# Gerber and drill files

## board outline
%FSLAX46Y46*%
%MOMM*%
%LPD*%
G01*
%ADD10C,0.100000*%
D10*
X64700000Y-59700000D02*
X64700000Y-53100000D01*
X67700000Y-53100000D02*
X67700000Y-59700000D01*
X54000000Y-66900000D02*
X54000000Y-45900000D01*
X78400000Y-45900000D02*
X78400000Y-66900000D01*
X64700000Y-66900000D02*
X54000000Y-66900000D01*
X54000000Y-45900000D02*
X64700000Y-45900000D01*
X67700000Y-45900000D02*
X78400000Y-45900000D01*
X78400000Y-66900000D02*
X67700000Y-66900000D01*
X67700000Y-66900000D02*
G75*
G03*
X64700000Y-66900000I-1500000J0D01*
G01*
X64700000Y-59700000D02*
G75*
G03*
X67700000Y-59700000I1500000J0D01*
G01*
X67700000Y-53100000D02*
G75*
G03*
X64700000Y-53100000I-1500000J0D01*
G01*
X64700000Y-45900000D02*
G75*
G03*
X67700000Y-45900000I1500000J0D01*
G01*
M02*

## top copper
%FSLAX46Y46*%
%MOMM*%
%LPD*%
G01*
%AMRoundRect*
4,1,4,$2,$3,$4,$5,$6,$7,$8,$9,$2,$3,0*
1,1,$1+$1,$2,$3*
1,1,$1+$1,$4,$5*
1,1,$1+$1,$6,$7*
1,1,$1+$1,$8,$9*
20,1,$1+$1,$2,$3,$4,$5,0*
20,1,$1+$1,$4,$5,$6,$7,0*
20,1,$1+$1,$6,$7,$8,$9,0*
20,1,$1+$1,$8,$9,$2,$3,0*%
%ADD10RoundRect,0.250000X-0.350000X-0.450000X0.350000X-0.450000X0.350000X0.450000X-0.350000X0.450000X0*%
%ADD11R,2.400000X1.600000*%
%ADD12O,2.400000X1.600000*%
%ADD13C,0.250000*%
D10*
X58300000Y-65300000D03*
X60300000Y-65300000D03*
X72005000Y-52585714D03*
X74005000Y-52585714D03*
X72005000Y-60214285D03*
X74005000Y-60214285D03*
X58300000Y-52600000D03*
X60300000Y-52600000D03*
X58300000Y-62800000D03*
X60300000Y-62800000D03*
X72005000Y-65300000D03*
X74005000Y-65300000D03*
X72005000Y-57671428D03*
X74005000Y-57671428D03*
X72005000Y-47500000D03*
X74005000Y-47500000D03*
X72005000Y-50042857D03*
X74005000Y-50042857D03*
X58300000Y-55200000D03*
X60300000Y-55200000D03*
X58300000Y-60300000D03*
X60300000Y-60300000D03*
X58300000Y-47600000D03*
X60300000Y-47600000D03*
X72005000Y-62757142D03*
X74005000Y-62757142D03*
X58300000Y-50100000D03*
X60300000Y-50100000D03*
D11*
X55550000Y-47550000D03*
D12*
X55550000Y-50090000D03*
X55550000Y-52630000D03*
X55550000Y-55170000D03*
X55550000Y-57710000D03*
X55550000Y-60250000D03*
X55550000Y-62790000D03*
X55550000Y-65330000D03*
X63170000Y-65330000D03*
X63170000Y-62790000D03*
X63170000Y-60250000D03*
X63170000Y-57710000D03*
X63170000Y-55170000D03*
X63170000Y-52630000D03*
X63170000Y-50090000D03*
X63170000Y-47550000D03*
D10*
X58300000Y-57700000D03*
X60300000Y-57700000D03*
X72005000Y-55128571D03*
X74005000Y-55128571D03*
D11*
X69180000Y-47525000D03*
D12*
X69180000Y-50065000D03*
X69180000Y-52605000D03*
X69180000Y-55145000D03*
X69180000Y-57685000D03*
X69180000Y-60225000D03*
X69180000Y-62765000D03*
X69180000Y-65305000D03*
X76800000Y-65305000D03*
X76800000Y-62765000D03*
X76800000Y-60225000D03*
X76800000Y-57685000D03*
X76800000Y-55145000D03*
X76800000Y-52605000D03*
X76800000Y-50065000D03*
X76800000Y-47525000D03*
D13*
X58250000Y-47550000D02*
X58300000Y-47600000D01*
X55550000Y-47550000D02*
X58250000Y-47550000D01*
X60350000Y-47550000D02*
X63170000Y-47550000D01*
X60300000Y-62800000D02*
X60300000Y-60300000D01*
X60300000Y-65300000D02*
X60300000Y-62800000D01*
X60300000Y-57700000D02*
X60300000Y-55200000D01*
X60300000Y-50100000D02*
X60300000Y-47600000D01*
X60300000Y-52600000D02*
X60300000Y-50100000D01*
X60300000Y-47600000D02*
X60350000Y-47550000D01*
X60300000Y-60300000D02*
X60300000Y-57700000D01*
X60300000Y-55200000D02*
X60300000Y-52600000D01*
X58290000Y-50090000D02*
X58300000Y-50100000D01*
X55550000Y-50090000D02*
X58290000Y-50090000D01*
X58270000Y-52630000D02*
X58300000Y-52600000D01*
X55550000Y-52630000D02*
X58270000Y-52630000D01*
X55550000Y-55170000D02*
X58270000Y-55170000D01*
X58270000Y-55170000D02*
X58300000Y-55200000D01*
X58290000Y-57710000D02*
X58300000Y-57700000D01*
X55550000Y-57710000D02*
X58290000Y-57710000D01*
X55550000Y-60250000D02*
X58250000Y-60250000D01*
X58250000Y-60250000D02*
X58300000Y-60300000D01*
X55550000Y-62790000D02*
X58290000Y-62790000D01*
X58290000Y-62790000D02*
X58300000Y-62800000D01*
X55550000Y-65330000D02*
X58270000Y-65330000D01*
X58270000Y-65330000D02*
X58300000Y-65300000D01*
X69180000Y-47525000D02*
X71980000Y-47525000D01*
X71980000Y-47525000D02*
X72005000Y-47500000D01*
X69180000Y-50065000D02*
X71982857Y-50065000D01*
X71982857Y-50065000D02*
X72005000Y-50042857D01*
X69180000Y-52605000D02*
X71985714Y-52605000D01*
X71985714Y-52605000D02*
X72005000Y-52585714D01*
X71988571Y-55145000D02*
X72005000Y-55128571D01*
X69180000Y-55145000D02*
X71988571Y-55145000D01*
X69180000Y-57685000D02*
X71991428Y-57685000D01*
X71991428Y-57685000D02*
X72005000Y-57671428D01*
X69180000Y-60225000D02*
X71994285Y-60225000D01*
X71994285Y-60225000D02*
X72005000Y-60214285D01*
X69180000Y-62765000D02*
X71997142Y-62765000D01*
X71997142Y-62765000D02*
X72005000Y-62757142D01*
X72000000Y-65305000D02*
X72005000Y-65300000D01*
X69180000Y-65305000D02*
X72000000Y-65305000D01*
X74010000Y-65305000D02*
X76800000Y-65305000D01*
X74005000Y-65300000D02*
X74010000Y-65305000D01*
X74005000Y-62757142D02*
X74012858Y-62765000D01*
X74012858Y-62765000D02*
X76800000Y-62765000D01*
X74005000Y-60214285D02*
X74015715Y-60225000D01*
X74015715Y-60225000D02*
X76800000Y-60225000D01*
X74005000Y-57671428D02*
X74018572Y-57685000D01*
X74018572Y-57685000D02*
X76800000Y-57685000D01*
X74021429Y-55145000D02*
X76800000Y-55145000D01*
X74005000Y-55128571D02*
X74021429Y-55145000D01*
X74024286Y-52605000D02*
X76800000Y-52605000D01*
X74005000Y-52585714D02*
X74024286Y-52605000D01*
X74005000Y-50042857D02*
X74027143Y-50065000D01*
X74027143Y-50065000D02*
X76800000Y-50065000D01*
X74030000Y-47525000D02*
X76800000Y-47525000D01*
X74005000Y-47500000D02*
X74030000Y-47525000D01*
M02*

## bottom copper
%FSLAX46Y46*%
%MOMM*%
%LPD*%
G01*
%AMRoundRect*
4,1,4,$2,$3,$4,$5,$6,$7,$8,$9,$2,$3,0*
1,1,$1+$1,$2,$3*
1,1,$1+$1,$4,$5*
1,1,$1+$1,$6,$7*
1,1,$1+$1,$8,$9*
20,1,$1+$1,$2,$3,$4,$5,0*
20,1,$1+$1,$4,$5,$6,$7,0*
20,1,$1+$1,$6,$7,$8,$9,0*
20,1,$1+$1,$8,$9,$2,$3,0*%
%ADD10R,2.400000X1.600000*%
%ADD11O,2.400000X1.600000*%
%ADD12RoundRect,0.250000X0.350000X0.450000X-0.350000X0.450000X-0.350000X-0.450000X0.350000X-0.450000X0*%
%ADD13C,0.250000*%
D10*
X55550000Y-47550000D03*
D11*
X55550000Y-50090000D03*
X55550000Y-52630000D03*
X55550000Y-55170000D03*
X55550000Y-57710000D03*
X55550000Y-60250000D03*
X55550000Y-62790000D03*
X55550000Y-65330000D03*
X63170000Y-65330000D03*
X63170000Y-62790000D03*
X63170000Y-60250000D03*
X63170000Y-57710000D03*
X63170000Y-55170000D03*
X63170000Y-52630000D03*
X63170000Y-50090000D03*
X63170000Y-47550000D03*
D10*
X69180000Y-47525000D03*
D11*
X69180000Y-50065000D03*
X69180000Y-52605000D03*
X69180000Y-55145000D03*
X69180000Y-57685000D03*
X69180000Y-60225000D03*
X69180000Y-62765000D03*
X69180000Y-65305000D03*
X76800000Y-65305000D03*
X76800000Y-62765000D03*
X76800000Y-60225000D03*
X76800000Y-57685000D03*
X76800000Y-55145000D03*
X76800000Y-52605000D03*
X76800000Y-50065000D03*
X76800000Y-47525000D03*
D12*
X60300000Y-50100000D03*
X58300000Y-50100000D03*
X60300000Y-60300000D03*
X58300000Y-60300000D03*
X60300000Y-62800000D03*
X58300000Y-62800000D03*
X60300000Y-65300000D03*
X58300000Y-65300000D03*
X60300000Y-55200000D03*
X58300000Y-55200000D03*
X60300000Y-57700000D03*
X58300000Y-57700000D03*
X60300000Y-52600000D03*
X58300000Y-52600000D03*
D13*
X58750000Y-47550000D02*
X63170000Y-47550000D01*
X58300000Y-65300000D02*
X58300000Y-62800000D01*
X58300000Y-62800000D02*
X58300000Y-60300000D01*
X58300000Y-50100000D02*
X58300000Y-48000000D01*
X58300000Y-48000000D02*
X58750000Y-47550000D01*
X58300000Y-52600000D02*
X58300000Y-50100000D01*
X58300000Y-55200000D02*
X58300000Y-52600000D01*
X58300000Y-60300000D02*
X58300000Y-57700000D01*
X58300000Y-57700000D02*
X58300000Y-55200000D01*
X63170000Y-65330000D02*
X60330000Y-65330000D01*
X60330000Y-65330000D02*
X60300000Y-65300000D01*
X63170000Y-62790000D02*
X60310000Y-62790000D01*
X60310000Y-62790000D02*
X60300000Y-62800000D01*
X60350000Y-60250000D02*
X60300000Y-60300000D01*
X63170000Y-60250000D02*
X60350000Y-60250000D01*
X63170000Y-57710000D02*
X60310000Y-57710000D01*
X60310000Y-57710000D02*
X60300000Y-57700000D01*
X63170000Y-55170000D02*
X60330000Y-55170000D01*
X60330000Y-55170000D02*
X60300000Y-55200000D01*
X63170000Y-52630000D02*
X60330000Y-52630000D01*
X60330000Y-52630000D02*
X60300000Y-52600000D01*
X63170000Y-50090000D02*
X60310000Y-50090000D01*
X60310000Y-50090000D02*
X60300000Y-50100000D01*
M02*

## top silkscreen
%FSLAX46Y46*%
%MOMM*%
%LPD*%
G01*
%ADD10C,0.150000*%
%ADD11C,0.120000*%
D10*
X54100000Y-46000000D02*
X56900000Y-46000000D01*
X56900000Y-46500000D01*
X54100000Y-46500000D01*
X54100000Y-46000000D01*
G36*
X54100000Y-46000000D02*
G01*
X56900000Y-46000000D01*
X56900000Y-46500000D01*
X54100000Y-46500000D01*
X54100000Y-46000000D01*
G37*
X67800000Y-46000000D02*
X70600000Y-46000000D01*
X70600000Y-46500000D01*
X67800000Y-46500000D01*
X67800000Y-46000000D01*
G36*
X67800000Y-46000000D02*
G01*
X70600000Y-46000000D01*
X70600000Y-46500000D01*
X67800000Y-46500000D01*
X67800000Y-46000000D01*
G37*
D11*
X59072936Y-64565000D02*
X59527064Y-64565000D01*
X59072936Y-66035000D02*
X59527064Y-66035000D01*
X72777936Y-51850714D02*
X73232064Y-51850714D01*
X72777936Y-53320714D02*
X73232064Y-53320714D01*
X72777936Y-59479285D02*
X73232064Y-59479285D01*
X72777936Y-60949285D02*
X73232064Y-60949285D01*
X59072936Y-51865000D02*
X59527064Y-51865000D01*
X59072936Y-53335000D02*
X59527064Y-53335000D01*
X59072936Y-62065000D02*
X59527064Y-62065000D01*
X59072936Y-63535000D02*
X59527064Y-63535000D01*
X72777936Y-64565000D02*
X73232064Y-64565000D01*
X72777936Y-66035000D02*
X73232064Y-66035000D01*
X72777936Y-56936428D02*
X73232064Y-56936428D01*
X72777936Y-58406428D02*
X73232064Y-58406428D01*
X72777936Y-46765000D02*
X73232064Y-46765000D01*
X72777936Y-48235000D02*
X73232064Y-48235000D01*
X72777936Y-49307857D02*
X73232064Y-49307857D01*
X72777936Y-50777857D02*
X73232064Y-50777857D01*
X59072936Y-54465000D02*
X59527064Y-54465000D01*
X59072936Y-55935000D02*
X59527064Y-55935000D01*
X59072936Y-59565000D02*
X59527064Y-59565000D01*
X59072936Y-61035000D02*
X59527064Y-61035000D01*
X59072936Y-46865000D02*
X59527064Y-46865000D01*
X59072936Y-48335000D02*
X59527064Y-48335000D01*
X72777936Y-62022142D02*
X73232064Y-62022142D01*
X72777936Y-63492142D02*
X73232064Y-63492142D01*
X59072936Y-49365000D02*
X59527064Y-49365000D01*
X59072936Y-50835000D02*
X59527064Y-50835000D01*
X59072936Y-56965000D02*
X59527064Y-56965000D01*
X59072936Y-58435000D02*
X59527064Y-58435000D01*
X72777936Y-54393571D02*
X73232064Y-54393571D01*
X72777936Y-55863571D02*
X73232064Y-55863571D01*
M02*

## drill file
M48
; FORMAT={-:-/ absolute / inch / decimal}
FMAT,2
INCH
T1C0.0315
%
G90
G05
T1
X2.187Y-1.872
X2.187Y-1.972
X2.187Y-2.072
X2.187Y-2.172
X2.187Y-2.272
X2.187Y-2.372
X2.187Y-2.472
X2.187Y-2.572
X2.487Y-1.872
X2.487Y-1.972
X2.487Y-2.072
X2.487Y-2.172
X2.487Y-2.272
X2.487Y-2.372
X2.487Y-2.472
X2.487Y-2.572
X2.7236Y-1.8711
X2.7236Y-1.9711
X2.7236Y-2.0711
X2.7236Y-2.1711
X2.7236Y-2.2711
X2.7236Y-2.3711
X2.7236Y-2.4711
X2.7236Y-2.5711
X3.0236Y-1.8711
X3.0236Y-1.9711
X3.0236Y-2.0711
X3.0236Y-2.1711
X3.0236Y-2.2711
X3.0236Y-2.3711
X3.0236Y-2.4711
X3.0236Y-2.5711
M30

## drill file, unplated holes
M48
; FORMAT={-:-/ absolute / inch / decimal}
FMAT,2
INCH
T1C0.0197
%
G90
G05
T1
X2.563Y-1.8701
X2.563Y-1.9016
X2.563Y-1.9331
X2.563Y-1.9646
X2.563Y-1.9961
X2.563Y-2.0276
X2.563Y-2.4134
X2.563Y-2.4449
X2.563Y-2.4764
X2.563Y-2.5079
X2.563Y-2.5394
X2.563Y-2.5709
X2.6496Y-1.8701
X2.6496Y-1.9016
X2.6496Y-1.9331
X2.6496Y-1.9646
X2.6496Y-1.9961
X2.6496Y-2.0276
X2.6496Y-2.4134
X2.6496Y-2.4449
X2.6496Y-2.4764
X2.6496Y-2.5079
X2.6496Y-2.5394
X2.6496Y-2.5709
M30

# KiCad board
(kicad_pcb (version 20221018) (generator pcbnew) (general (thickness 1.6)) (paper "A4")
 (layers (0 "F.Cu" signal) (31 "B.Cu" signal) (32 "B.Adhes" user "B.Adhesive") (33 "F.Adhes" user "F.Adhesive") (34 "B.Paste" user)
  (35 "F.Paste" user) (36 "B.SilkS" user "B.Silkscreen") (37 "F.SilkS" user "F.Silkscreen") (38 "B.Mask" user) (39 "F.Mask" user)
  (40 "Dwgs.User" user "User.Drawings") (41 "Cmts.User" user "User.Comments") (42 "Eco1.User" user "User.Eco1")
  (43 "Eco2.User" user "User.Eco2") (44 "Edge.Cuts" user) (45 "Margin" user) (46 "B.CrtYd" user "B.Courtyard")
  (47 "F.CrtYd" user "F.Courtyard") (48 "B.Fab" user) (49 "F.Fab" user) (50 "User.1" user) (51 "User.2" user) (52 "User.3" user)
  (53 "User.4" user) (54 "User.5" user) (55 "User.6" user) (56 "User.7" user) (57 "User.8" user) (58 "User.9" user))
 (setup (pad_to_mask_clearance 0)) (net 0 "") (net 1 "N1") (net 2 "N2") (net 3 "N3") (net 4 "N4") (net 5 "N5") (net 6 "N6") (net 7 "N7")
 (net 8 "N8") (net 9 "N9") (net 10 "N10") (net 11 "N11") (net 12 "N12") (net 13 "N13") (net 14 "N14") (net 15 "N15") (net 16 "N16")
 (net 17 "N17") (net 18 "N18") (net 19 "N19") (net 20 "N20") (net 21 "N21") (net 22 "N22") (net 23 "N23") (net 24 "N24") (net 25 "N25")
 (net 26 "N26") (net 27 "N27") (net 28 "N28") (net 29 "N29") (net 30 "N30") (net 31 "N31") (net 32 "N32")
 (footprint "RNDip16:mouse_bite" (layer "F.Cu") (at 66.2 63.3 90)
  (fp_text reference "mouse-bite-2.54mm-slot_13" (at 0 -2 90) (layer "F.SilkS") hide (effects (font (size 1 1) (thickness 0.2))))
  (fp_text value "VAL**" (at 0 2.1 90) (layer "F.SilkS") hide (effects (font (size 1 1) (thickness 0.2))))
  (fp_arc (start -3.6 -1.5) (mid -2.1 0) (end -3.6 1.5) (stroke (width 0.1) (type solid)) (layer "Edge.Cuts"))
  (fp_arc (start 3.6 1.5) (mid 2.1 0) (end 3.6 -1.5) (stroke (width 0.1) (type solid)) (layer "Edge.Cuts"))
  (pad "" np_thru_hole circle (at -2 -1.1 90) (size 0.5 0.5) (drill 0.5) (layers "F&B.Cu" "*.Mask"))
  (pad "" np_thru_hole circle (at -2 1.1 90) (size 0.5 0.5) (drill 0.5) (layers "F&B.Cu" "*.Mask"))
  (pad "" np_thru_hole circle (at -1.2 -1.1 90) (size 0.5 0.5) (drill 0.5) (layers "F&B.Cu" "*.Mask"))
  (pad "" np_thru_hole circle (at -1.2 1.1 90) (size 0.5 0.5) (drill 0.5) (layers "F&B.Cu" "*.Mask"))
  (pad "" np_thru_hole circle (at -0.4 -1.1 90) (size 0.5 0.5) (drill 0.5) (layers "F&B.Cu" "*.Mask"))
  (pad "" np_thru_hole circle (at -0.4 1.1 90) (size 0.5 0.5) (drill 0.5) (layers "F&B.Cu" "*.Mask"))
  (pad "" np_thru_hole circle (at 0.4 -1.1 90) (size 0.5 0.5) (drill 0.5) (layers "F&B.Cu" "*.Mask"))
  (pad "" np_thru_hole circle (at 0.4 1.1 90) (size 0.5 0.5) (drill 0.5) (layers "F&B.Cu" "*.Mask"))
  (pad "" np_thru_hole circle (at 1.2 -1.1 90) (size 0.5 0.5) (drill 0.5) (layers "F&B.Cu" "*.Mask"))
  (pad "" np_thru_hole circle (at 1.2 1.1 90) (size 0.5 0.5) (drill 0.5) (layers "F&B.Cu" "*.Mask"))
  (pad "" np_thru_hole circle (at 2 -1.1 90) (size 0.5 0.5) (drill 0.5) (layers "F&B.Cu" "*.Mask"))
  (pad "" np_thru_hole circle (at 2 1.1 90) (size 0.5 0.5) (drill 0.5) (layers "F&B.Cu" "*.Mask")))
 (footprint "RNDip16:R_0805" (layer "F.Cu") (at 59.3 65.3)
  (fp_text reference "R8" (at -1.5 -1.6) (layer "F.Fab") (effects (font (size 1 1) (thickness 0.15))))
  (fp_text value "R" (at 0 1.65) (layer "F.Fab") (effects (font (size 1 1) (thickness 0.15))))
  (fp_line (start -0.227064 -0.735) (end 0.227064 -0.735) (stroke (width 0.12) (type solid)) (layer "F.SilkS"))
  (fp_line (start -0.227064 0.735) (end 0.227064 0.735) (stroke (width 0.12) (type solid)) (layer "F.SilkS"))
  (pad "1" smd roundrect (at -1 0) (size 1.2 1.4) (layers "F.Cu" "F.Paste" "F.Mask") (roundrect_rratio 0.2083333333) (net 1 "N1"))
  (pad "2" smd roundrect (at 1 0) (size 1.2 1.4) (layers "F.Cu" "F.Paste" "F.Mask") (roundrect_rratio 0.2083333333) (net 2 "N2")))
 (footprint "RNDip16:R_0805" (layer "F.Cu") (at 73.005 52.585714)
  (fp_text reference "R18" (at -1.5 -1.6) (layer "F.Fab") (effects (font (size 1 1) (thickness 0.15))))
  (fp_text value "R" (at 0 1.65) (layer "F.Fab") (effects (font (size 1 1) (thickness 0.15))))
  (fp_line (start -0.227064 -0.735) (end 0.227064 -0.735) (stroke (width 0.12) (type solid)) (layer "F.SilkS"))
  (fp_line (start -0.227064 0.735) (end 0.227064 0.735) (stroke (width 0.12) (type solid)) (layer "F.SilkS"))
  (pad "1" smd roundrect (at -1 0) (size 1.2 1.4) (layers "F.Cu" "F.Paste" "F.Mask") (roundrect_rratio 0.2083333333) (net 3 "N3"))
  (pad "2" smd roundrect (at 1 0) (size 1.2 1.4) (layers "F.Cu" "F.Paste" "F.Mask") (roundrect_rratio 0.2083333333) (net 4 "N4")))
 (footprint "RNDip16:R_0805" (layer "F.Cu") (at 73.005 60.214285)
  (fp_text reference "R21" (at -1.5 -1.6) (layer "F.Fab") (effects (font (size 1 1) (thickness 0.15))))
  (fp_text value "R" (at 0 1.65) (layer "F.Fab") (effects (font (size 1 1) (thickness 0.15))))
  (fp_line (start -0.227064 -0.735) (end 0.227064 -0.735) (stroke (width 0.12) (type solid)) (layer "F.SilkS"))
  (fp_line (start -0.227064 0.735) (end 0.227064 0.735) (stroke (width 0.12) (type solid)) (layer "F.SilkS"))
  (pad "1" smd roundrect (at -1 0) (size 1.2 1.4) (layers "F.Cu" "F.Paste" "F.Mask") (roundrect_rratio 0.2083333333) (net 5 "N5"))
  (pad "2" smd roundrect (at 1 0) (size 1.2 1.4) (layers "F.Cu" "F.Paste" "F.Mask") (roundrect_rratio 0.2083333333) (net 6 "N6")))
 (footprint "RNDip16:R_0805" (layer "F.Cu") (at 59.3 52.6)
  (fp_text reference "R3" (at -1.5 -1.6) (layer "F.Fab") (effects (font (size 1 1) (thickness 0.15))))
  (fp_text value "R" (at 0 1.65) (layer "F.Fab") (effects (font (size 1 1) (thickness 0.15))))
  (fp_line (start -0.227064 -0.735) (end 0.227064 -0.735) (stroke (width 0.12) (type solid)) (layer "F.SilkS"))
  (fp_line (start -0.227064 0.735) (end 0.227064 0.735) (stroke (width 0.12) (type solid)) (layer "F.SilkS"))
  (pad "1" smd roundrect (at -1 0) (size 1.2 1.4) (layers "F.Cu" "F.Paste" "F.Mask") (roundrect_rratio 0.2083333333) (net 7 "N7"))
  (pad "2" smd roundrect (at 1 0) (size 1.2 1.4) (layers "F.Cu" "F.Paste" "F.Mask") (roundrect_rratio 0.2083333333) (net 2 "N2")))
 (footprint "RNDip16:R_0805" (layer "F.Cu") (at 59.3 62.8)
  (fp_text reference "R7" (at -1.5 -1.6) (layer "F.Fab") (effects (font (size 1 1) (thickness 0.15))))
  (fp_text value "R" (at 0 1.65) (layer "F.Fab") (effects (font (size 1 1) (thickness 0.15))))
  (fp_line (start -0.227064 -0.735) (end 0.227064 -0.735) (stroke (width 0.12) (type solid)) (layer "F.SilkS"))
  (fp_line (start -0.227064 0.735) (end 0.227064 0.735) (stroke (width 0.12) (type solid)) (layer "F.SilkS"))
  (pad "1" smd roundrect (at -1 0) (size 1.2 1.4) (layers "F.Cu" "F.Paste" "F.Mask") (roundrect_rratio 0.2083333333) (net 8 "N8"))
  (pad "2" smd roundrect (at 1 0) (size 1.2 1.4) (layers "F.Cu" "F.Paste" "F.Mask") (roundrect_rratio 0.2083333333) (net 2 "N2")))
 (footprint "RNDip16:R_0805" (layer "F.Cu") (at 73.005 65.3)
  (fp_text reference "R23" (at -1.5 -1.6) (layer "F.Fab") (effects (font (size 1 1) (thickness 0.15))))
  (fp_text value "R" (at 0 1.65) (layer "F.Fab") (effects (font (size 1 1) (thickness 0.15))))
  (fp_line (start -0.227064 -0.735) (end 0.227064 -0.735) (stroke (width 0.12) (type solid)) (layer "F.SilkS"))
  (fp_line (start -0.227064 0.735) (end 0.227064 0.735) (stroke (width 0.12) (type solid)) (layer "F.SilkS"))
  (pad "1" smd roundrect (at -1 0) (size 1.2 1.4) (layers "F.Cu" "F.Paste" "F.Mask") (roundrect_rratio 0.2083333333) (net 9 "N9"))
  (pad "2" smd roundrect (at 1 0) (size 1.2 1.4) (layers "F.Cu" "F.Paste" "F.Mask") (roundrect_rratio 0.2083333333) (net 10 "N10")))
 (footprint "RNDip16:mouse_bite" (layer "F.Cu") (at 66.2 49.5 90)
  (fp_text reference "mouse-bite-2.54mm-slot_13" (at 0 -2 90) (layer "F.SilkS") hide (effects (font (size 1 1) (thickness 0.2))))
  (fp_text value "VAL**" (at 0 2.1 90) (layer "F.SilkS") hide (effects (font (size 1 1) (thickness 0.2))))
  (fp_arc (start -3.6 -1.5) (mid -2.1 0) (end -3.6 1.5) (stroke (width 0.1) (type solid)) (layer "Edge.Cuts"))
  (fp_arc (start 3.6 1.5) (mid 2.1 0) (end 3.6 -1.5) (stroke (width 0.1) (type solid)) (layer "Edge.Cuts"))
  (pad "" np_thru_hole circle (at -2 -1.1 90) (size 0.5 0.5) (drill 0.5) (layers "F&B.Cu" "*.Mask"))
  (pad "" np_thru_hole circle (at -2 1.1 90) (size 0.5 0.5) (drill 0.5) (layers "F&B.Cu" "*.Mask"))
  (pad "" np_thru_hole circle (at -1.2 -1.1 90) (size 0.5 0.5) (drill 0.5) (layers "F&B.Cu" "*.Mask"))
  (pad "" np_thru_hole circle (at -1.2 1.1 90) (size 0.5 0.5) (drill 0.5) (layers "F&B.Cu" "*.Mask"))
  (pad "" np_thru_hole circle (at -0.4 -1.1 90) (size 0.5 0.5) (drill 0.5) (layers "F&B.Cu" "*.Mask"))
  (pad "" np_thru_hole circle (at -0.4 1.1 90) (size 0.5 0.5) (drill 0.5) (layers "F&B.Cu" "*.Mask"))
  (pad "" np_thru_hole circle (at 0.4 -1.1 90) (size 0.5 0.5) (drill 0.5) (layers "F&B.Cu" "*.Mask"))
  (pad "" np_thru_hole circle (at 0.4 1.1 90) (size 0.5 0.5) (drill 0.5) (layers "F&B.Cu" "*.Mask"))
  (pad "" np_thru_hole circle (at 1.2 -1.1 90) (size 0.5 0.5) (drill 0.5) (layers "F&B.Cu" "*.Mask"))
  (pad "" np_thru_hole circle (at 1.2 1.1 90) (size 0.5 0.5) (drill 0.5) (layers "F&B.Cu" "*.Mask"))
  (pad "" np_thru_hole circle (at 2 -1.1 90) (size 0.5 0.5) (drill 0.5) (layers "F&B.Cu" "*.Mask"))
  (pad "" np_thru_hole circle (at 2 1.1 90) (size 0.5 0.5) (drill 0.5) (layers "F&B.Cu" "*.Mask")))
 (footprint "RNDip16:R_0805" (layer "F.Cu") (at 73.005 57.671428)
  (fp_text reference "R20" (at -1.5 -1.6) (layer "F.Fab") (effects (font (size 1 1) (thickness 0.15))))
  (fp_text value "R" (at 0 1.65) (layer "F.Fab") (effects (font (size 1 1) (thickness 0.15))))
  (fp_line (start -0.227064 -0.735) (end 0.227064 -0.735) (stroke (width 0.12) (type solid)) (layer "F.SilkS"))
  (fp_line (start -0.227064 0.735) (end 0.227064 0.735) (stroke (width 0.12) (type solid)) (layer "F.SilkS"))
  (pad "1" smd roundrect (at -1 0) (size 1.2 1.4) (layers "F.Cu" "F.Paste" "F.Mask") (roundrect_rratio 0.2083333333) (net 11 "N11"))
  (pad "2" smd roundrect (at 1 0) (size 1.2 1.4) (layers "F.Cu" "F.Paste" "F.Mask") (roundrect_rratio 0.2083333333) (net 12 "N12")))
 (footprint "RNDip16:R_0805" (layer "F.Cu") (at 73.005 47.5)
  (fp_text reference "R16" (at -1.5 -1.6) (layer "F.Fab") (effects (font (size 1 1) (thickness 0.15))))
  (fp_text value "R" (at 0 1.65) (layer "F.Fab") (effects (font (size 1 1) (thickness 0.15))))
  (fp_line (start -0.227064 -0.735) (end 0.227064 -0.735) (stroke (width 0.12) (type solid)) (layer "F.SilkS"))
  (fp_line (start -0.227064 0.735) (end 0.227064 0.735) (stroke (width 0.12) (type solid)) (layer "F.SilkS"))
  (pad "1" smd roundrect (at -1 0) (size 1.2 1.4) (layers "F.Cu" "F.Paste" "F.Mask") (roundrect_rratio 0.2083333333) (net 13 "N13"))
  (pad "2" smd roundrect (at 1 0) (size 1.2 1.4) (layers "F.Cu" "F.Paste" "F.Mask") (roundrect_rratio 0.2083333333) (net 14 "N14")))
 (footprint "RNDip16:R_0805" (layer "F.Cu") (at 73.005 50.042857)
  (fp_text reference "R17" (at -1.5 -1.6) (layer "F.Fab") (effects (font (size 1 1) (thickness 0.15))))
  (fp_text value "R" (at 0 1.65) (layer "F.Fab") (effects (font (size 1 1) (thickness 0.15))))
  (fp_line (start -0.227064 -0.735) (end 0.227064 -0.735) (stroke (width 0.12) (type solid)) (layer "F.SilkS"))
  (fp_line (start -0.227064 0.735) (end 0.227064 0.735) (stroke (width 0.12) (type solid)) (layer "F.SilkS"))
  (pad "1" smd roundrect (at -1 0) (size 1.2 1.4) (layers "F.Cu" "F.Paste" "F.Mask") (roundrect_rratio 0.2083333333) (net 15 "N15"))
  (pad "2" smd roundrect (at 1 0) (size 1.2 1.4) (layers "F.Cu" "F.Paste" "F.Mask") (roundrect_rratio 0.2083333333) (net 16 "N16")))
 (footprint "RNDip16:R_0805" (layer "F.Cu") (at 59.3 55.2)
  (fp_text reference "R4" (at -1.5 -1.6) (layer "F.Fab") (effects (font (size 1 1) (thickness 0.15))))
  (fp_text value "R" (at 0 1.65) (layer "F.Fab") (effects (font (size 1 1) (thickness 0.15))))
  (fp_line (start -0.227064 -0.735) (end 0.227064 -0.735) (stroke (width 0.12) (type solid)) (layer "F.SilkS"))
  (fp_line (start -0.227064 0.735) (end 0.227064 0.735) (stroke (width 0.12) (type solid)) (layer "F.SilkS"))
  (pad "1" smd roundrect (at -1 0) (size 1.2 1.4) (layers "F.Cu" "F.Paste" "F.Mask") (roundrect_rratio 0.2083333333) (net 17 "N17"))
  (pad "2" smd roundrect (at 1 0) (size 1.2 1.4) (layers "F.Cu" "F.Paste" "F.Mask") (roundrect_rratio 0.2083333333) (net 2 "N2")))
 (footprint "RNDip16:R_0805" (layer "F.Cu") (at 59.3 60.3)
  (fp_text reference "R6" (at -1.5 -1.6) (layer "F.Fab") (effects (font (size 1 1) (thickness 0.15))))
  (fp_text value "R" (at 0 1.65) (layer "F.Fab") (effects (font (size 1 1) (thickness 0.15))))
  (fp_line (start -0.227064 -0.735) (end 0.227064 -0.735) (stroke (width 0.12) (type solid)) (layer "F.SilkS"))
  (fp_line (start -0.227064 0.735) (end 0.227064 0.735) (stroke (width 0.12) (type solid)) (layer "F.SilkS"))
  (pad "1" smd roundrect (at -1 0) (size 1.2 1.4) (layers "F.Cu" "F.Paste" "F.Mask") (roundrect_rratio 0.2083333333) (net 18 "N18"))
  (pad "2" smd roundrect (at 1 0) (size 1.2 1.4) (layers "F.Cu" "F.Paste" "F.Mask") (roundrect_rratio 0.2083333333) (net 2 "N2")))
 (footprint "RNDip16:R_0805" (layer "F.Cu") (at 59.3 47.6)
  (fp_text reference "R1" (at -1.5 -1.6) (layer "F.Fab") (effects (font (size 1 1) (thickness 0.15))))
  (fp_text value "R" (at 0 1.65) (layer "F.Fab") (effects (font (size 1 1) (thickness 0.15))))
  (fp_line (start -0.227064 -0.735) (end 0.227064 -0.735) (stroke (width 0.12) (type solid)) (layer "F.SilkS"))
  (fp_line (start -0.227064 0.735) (end 0.227064 0.735) (stroke (width 0.12) (type solid)) (layer "F.SilkS"))
  (pad "1" smd roundrect (at -1 0) (size 1.2 1.4) (layers "F.Cu" "F.Paste" "F.Mask") (roundrect_rratio 0.2083333333) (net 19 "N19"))
  (pad "2" smd roundrect (at 1 0) (size 1.2 1.4) (layers "F.Cu" "F.Paste" "F.Mask") (roundrect_rratio 0.2083333333) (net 2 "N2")))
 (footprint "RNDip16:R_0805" (layer "F.Cu") (at 73.005 62.757142)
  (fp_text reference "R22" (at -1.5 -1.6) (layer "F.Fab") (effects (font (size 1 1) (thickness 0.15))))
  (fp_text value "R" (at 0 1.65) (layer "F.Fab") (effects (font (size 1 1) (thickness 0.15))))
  (fp_line (start -0.227064 -0.735) (end 0.227064 -0.735) (stroke (width 0.12) (type solid)) (layer "F.SilkS"))
  (fp_line (start -0.227064 0.735) (end 0.227064 0.735) (stroke (width 0.12) (type solid)) (layer "F.SilkS"))
  (pad "1" smd roundrect (at -1 0) (size 1.2 1.4) (layers "F.Cu" "F.Paste" "F.Mask") (roundrect_rratio 0.2083333333) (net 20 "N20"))
  (pad "2" smd roundrect (at 1 0) (size 1.2 1.4) (layers "F.Cu" "F.Paste" "F.Mask") (roundrect_rratio 0.2083333333) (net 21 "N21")))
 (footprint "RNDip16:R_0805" (layer "F.Cu") (at 59.3 50.1)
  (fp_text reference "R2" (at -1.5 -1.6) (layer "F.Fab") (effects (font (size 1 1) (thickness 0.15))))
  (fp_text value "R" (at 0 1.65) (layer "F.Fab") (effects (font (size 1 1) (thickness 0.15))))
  (fp_line (start -0.227064 -0.735) (end 0.227064 -0.735) (stroke (width 0.12) (type solid)) (layer "F.SilkS"))
  (fp_line (start -0.227064 0.735) (end 0.227064 0.735) (stroke (width 0.12) (type solid)) (layer "F.SilkS"))
  (pad "1" smd roundrect (at -1 0) (size 1.2 1.4) (layers "F.Cu" "F.Paste" "F.Mask") (roundrect_rratio 0.2083333333) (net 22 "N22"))
  (pad "2" smd roundrect (at 1 0) (size 1.2 1.4) (layers "F.Cu" "F.Paste" "F.Mask") (roundrect_rratio 0.2083333333) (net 2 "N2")))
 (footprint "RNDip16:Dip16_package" (layer "F.Cu") (at 55.55 47.55)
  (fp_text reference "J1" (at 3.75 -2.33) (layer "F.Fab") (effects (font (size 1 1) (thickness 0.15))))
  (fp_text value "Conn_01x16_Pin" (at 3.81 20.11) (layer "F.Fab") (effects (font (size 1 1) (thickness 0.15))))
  (pad "1" thru_hole rect (at 0 0) (size 2.4 1.6) (drill 0.8) (layers "*.Cu" "*.Mask") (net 19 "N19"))
  (pad "2" thru_hole oval (at 0 2.54) (size 2.4 1.6) (drill 0.8) (layers "*.Cu" "*.Mask") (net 22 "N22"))
  (pad "3" thru_hole oval (at 0 5.08) (size 2.4 1.6) (drill 0.8) (layers "*.Cu" "*.Mask") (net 7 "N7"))
  (pad "4" thru_hole oval (at 0 7.62) (size 2.4 1.6) (drill 0.8) (layers "*.Cu" "*.Mask") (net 17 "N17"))
  (pad "5" thru_hole oval (at 0 10.16) (size 2.4 1.6) (drill 0.8) (layers "*.Cu" "*.Mask") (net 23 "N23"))
  (pad "6" thru_hole oval (at 0 12.7) (size 2.4 1.6) (drill 0.8) (layers "*.Cu" "*.Mask") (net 18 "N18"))
  (pad "7" thru_hole oval (at 0 15.24) (size 2.4 1.6) (drill 0.8) (layers "*.Cu" "*.Mask") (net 8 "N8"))
  (pad "8" thru_hole oval (at 0 17.78) (size 2.4 1.6) (drill 0.8) (layers "*.Cu" "*.Mask") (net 1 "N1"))
  (pad "9" thru_hole oval (at 7.62 17.78) (size 2.4 1.6) (drill 0.8) (layers "*.Cu" "*.Mask") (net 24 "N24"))
  (pad "10" thru_hole oval (at 7.62 15.24) (size 2.4 1.6) (drill 0.8) (layers "*.Cu" "*.Mask") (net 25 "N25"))
  (pad "11" thru_hole oval (at 7.62 12.7) (size 2.4 1.6) (drill 0.8) (layers "*.Cu" "*.Mask") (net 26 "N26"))
  (pad "12" thru_hole oval (at 7.62 10.16) (size 2.4 1.6) (drill 0.8) (layers "*.Cu" "*.Mask") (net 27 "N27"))
  (pad "13" thru_hole oval (at 7.62 7.62) (size 2.4 1.6) (drill 0.8) (layers "*.Cu" "*.Mask") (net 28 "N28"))
  (pad "14" thru_hole oval (at 7.62 5.08) (size 2.4 1.6) (drill 0.8) (layers "*.Cu" "*.Mask") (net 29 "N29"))
  (pad "15" thru_hole oval (at 7.62 2.54) (size 2.4 1.6) (drill 0.8) (layers "*.Cu" "*.Mask") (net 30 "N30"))
  (pad "16" thru_hole oval (at 7.62 0) (size 2.4 1.6) (drill 0.8) (layers "*.Cu" "*.Mask") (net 2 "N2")))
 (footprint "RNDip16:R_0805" (layer "F.Cu") (at 59.3 57.7)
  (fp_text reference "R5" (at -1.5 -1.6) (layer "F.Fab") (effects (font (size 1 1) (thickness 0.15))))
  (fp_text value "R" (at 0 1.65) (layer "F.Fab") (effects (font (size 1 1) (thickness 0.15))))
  (fp_line (start -0.227064 -0.735) (end 0.227064 -0.735) (stroke (width 0.12) (type solid)) (layer "F.SilkS"))
  (fp_line (start -0.227064 0.735) (end 0.227064 0.735) (stroke (width 0.12) (type solid)) (layer "F.SilkS"))
  (pad "1" smd roundrect (at -1 0) (size 1.2 1.4) (layers "F.Cu" "F.Paste" "F.Mask") (roundrect_rratio 0.2083333333) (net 23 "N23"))
  (pad "2" smd roundrect (at 1 0) (size 1.2 1.4) (layers "F.Cu" "F.Paste" "F.Mask") (roundrect_rratio 0.2083333333) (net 2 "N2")))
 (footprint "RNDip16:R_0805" (layer "F.Cu") (at 73.005 55.128571)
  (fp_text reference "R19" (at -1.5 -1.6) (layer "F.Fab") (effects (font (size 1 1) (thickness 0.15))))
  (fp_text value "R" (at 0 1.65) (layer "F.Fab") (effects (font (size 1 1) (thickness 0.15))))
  (fp_line (start -0.227064 -0.735) (end 0.227064 -0.735) (stroke (width 0.12) (type solid)) (layer "F.SilkS"))
  (fp_line (start -0.227064 0.735) (end 0.227064 0.735) (stroke (width 0.12) (type solid)) (layer "F.SilkS"))
  (pad "1" smd roundrect (at -1 0) (size 1.2 1.4) (layers "F.Cu" "F.Paste" "F.Mask") (roundrect_rratio 0.2083333333) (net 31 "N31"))
  (pad "2" smd roundrect (at 1 0) (size 1.2 1.4) (layers "F.Cu" "F.Paste" "F.Mask") (roundrect_rratio 0.2083333333) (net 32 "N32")))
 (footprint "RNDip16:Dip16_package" (layer "F.Cu") (at 69.18 47.525)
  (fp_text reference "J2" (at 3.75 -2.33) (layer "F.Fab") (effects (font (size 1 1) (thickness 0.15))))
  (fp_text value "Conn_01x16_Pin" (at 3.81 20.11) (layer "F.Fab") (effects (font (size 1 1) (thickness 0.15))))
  (pad "1" thru_hole rect (at 0 0) (size 2.4 1.6) (drill 0.8) (layers "*.Cu" "*.Mask") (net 13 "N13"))
  (pad "2" thru_hole oval (at 0 2.54) (size 2.4 1.6) (drill 0.8) (layers "*.Cu" "*.Mask") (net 15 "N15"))
  (pad "3" thru_hole oval (at 0 5.08) (size 2.4 1.6) (drill 0.8) (layers "*.Cu" "*.Mask") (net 3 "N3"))
  (pad "4" thru_hole oval (at 0 7.62) (size 2.4 1.6) (drill 0.8) (layers "*.Cu" "*.Mask") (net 31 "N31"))
  (pad "5" thru_hole oval (at 0 10.16) (size 2.4 1.6) (drill 0.8) (layers "*.Cu" "*.Mask") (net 11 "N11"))
  (pad "6" thru_hole oval (at 0 12.7) (size 2.4 1.6) (drill 0.8) (layers "*.Cu" "*.Mask") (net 5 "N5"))
  (pad "7" thru_hole oval (at 0 15.24) (size 2.4 1.6) (drill 0.8) (layers "*.Cu" "*.Mask") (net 20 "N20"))
  (pad "8" thru_hole oval (at 0 17.78) (size 2.4 1.6) (drill 0.8) (layers "*.Cu" "*.Mask") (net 9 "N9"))
  (pad "9" thru_hole oval (at 7.62 17.78) (size 2.4 1.6) (drill 0.8) (layers "*.Cu" "*.Mask") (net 10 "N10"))
  (pad "10" thru_hole oval (at 7.62 15.24) (size 2.4 1.6) (drill 0.8) (layers "*.Cu" "*.Mask") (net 21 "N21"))
  (pad "11" thru_hole oval (at 7.62 12.7) (size 2.4 1.6) (drill 0.8) (layers "*.Cu" "*.Mask") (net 6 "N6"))
  (pad "12" thru_hole oval (at 7.62 10.16) (size 2.4 1.6) (drill 0.8) (layers "*.Cu" "*.Mask") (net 12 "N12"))
  (pad "13" thru_hole oval (at 7.62 7.62) (size 2.4 1.6) (drill 0.8) (layers "*.Cu" "*.Mask") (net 32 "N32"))
  (pad "14" thru_hole oval (at 7.62 5.08) (size 2.4 1.6) (drill 0.8) (layers "*.Cu" "*.Mask") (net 4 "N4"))
  (pad "15" thru_hole oval (at 7.62 2.54) (size 2.4 1.6) (drill 0.8) (layers "*.Cu" "*.Mask") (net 16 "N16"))
  (pad "16" thru_hole oval (at 7.62 0) (size 2.4 1.6) (drill 0.8) (layers "*.Cu" "*.Mask") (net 14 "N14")))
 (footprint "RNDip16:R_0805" (layer "B.Cu") (at 59.3 50.1 180)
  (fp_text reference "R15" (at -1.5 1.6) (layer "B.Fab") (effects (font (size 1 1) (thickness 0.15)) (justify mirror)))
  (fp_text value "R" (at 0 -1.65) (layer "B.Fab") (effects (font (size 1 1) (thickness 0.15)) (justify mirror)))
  (pad "1" smd roundrect (at -1 0 180) (size 1.2 1.4) (layers "B.Cu" "B.Paste" "B.Mask") (roundrect_rratio 0.2083333333) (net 30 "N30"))
  (pad "2" smd roundrect (at 1 0 180) (size 1.2 1.4) (layers "B.Cu" "B.Paste" "B.Mask") (roundrect_rratio 0.2083333333) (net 2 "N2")))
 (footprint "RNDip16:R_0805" (layer "B.Cu") (at 59.3 60.3 180)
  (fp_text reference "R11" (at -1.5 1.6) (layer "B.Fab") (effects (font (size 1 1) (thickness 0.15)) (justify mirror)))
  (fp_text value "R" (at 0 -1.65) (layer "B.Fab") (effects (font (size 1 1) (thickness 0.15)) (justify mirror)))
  (pad "1" smd roundrect (at -1 0 180) (size 1.2 1.4) (layers "B.Cu" "B.Paste" "B.Mask") (roundrect_rratio 0.2083333333) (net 26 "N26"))
  (pad "2" smd roundrect (at 1 0 180) (size 1.2 1.4) (layers "B.Cu" "B.Paste" "B.Mask") (roundrect_rratio 0.2083333333) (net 2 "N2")))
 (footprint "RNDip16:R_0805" (layer "B.Cu") (at 59.3 62.8 180)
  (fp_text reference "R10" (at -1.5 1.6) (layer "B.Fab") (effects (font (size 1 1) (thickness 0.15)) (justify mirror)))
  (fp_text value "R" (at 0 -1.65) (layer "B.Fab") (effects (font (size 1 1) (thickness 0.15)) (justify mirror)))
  (pad "1" smd roundrect (at -1 0 180) (size 1.2 1.4) (layers "B.Cu" "B.Paste" "B.Mask") (roundrect_rratio 0.2083333333) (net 25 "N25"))
  (pad "2" smd roundrect (at 1 0 180) (size 1.2 1.4) (layers "B.Cu" "B.Paste" "B.Mask") (roundrect_rratio 0.2083333333) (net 2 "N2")))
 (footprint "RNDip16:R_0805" (layer "B.Cu") (at 59.3 65.3 180)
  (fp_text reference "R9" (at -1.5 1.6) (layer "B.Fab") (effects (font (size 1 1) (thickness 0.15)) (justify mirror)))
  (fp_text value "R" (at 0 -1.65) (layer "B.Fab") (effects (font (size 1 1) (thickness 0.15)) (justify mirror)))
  (pad "1" smd roundrect (at -1 0 180) (size 1.2 1.4) (layers "B.Cu" "B.Paste" "B.Mask") (roundrect_rratio 0.2083333333) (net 24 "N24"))
  (pad "2" smd roundrect (at 1 0 180) (size 1.2 1.4) (layers "B.Cu" "B.Paste" "B.Mask") (roundrect_rratio 0.2083333333) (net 2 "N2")))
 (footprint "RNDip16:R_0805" (layer "B.Cu") (at 59.3 55.2 180)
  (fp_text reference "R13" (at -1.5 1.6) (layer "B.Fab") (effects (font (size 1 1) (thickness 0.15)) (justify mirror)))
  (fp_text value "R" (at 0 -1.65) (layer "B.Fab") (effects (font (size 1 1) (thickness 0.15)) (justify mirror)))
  (pad "1" smd roundrect (at -1 0 180) (size 1.2 1.4) (layers "B.Cu" "B.Paste" "B.Mask") (roundrect_rratio 0.2083333333) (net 28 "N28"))
  (pad "2" smd roundrect (at 1 0 180) (size 1.2 1.4) (layers "B.Cu" "B.Paste" "B.Mask") (roundrect_rratio 0.2083333333) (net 2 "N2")))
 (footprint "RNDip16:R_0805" (layer "B.Cu") (at 59.3 57.7 180)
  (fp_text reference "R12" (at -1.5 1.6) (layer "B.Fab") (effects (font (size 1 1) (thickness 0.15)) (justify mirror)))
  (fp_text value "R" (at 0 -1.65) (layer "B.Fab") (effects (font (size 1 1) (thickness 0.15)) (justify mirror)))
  (pad "1" smd roundrect (at -1 0 180) (size 1.2 1.4) (layers "B.Cu" "B.Paste" "B.Mask") (roundrect_rratio 0.2083333333) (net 27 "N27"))
  (pad "2" smd roundrect (at 1 0 180) (size 1.2 1.4) (layers "B.Cu" "B.Paste" "B.Mask") (roundrect_rratio 0.2083333333) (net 2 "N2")))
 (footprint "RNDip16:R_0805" (layer "B.Cu") (at 59.3 52.6 180)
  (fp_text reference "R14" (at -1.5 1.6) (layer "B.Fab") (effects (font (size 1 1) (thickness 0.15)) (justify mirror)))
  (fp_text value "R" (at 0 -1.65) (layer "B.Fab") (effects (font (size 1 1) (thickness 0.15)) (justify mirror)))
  (pad "1" smd roundrect (at -1 0 180) (size 1.2 1.4) (layers "B.Cu" "B.Paste" "B.Mask") (roundrect_rratio 0.2083333333) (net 29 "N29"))
  (pad "2" smd roundrect (at 1 0 180) (size 1.2 1.4) (layers "B.Cu" "B.Paste" "B.Mask") (roundrect_rratio 0.2083333333) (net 2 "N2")))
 (gr_rect (start 54.1 46) (end 56.9 46.5) (stroke (width 0.15) (type solid)) (fill solid) (layer "F.SilkS"))
 (gr_rect (start 67.8 46) (end 70.6 46.5) (stroke (width 0.15) (type solid)) (fill solid) (layer "F.SilkS"))
 (gr_line (start 64.7 59.7) (end 64.7 53.1) (stroke (width 0.1) (type default)) (layer "Edge.Cuts"))
 (gr_line (start 67.7 53.1) (end 67.7 59.7) (stroke (width 0.1) (type default)) (layer "Edge.Cuts"))
 (gr_line (start 54 66.9) (end 54 45.9) (stroke (width 0.1) (type default)) (layer "Edge.Cuts"))
 (gr_line (start 78.4 45.9) (end 78.4 66.9) (stroke (width 0.1) (type default)) (layer "Edge.Cuts"))
 (gr_line (start 64.7 66.9) (end 54 66.9) (stroke (width 0.1) (type default)) (layer "Edge.Cuts"))
 (gr_line (start 54 45.9) (end 64.7 45.9) (stroke (width 0.1) (type default)) (layer "Edge.Cuts"))
 (gr_line (start 67.7 45.9) (end 78.4 45.9) (stroke (width 0.1) (type default)) (layer "Edge.Cuts"))
 (gr_line (start 78.4 66.9) (end 67.7 66.9) (stroke (width 0.1) (type default)) (layer "Edge.Cuts"))
 (segment (start 58.25 47.55) (end 58.3 47.6) (width 0.25) (layer "F.Cu") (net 19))
 (segment (start 55.55 47.55) (end 58.25 47.55) (width 0.25) (layer "F.Cu") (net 19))
 (segment (start 60.35 47.55) (end 63.17 47.55) (width 0.25) (layer "F.Cu") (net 2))
 (segment (start 60.3 62.8) (end 60.3 60.3) (width 0.25) (layer "F.Cu") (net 2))
 (segment (start 60.3 65.3) (end 60.3 62.8) (width 0.25) (layer "F.Cu") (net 2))
 (segment (start 60.3 57.7) (end 60.3 55.2) (width 0.25) (layer "F.Cu") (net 2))
 (segment (start 60.3 50.1) (end 60.3 47.6) (width 0.25) (layer "F.Cu") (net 2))
 (segment (start 60.3 52.6) (end 60.3 50.1) (width 0.25) (layer "F.Cu") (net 2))
 (segment (start 60.3 47.6) (end 60.35 47.55) (width 0.25) (layer "F.Cu") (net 2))
 (segment (start 60.3 60.3) (end 60.3 57.7) (width 0.25) (layer "F.Cu") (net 2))
 (segment (start 60.3 55.2) (end 60.3 52.6) (width 0.25) (layer "F.Cu") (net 2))
 (segment (start 58.75 47.55) (end 63.17 47.55) (width 0.25) (layer "B.Cu") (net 2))
 (segment (start 58.3 65.3) (end 58.3 62.8) (width 0.25) (layer "B.Cu") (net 2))
 (segment (start 58.3 62.8) (end 58.3 60.3) (width 0.25) (layer "B.Cu") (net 2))
 (segment (start 58.3 50.1) (end 58.3 48) (width 0.25) (layer "B.Cu") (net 2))
 (segment (start 58.3 48) (end 58.75 47.55) (width 0.25) (layer "B.Cu") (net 2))
 (segment (start 58.3 52.6) (end 58.3 50.1) (width 0.25) (layer "B.Cu") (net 2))
 (segment (start 58.3 55.2) (end 58.3 52.6) (width 0.25) (layer "B.Cu") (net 2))
 (segment (start 58.3 60.3) (end 58.3 57.7) (width 0.25) (layer "B.Cu") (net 2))
 (segment (start 58.3 57.7) (end 58.3 55.2) (width 0.25) (layer "B.Cu") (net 2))
 (segment (start 58.29 50.09) (end 58.3 50.1) (width 0.25) (layer "F.Cu") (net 22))
 (segment (start 55.55 50.09) (end 58.29 50.09) (width 0.25) (layer "F.Cu") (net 22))
 (segment (start 58.27 52.63) (end 58.3 52.6) (width 0.25) (layer "F.Cu") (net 7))
 (segment (start 55.55 52.63) (end 58.27 52.63) (width 0.25) (layer "F.Cu") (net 7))
 (segment (start 55.55 55.17) (end 58.27 55.17) (width 0.25) (layer "F.Cu") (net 17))
 (segment (start 58.27 55.17) (end 58.3 55.2) (width 0.25) (layer "F.Cu") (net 17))
 (segment (start 58.29 57.71) (end 58.3 57.7) (width 0.25) (layer "F.Cu") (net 23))
 (segment (start 55.55 57.71) (end 58.29 57.71) (width 0.25) (layer "F.Cu") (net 23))
 (segment (start 55.55 60.25) (end 58.25 60.25) (width 0.25) (layer "F.Cu") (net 18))
 (segment (start 58.25 60.25) (end 58.3 60.3) (width 0.25) (layer "F.Cu") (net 18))
 (segment (start 55.55 62.79) (end 58.29 62.79) (width 0.25) (layer "F.Cu") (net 8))
 (segment (start 58.29 62.79) (end 58.3 62.8) (width 0.25) (layer "F.Cu") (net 8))
 (segment (start 55.55 65.33) (end 58.27 65.33) (width 0.25) (layer "F.Cu") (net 1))
 (segment (start 58.27 65.33) (end 58.3 65.3) (width 0.25) (layer "F.Cu") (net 1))
 (segment (start 63.17 65.33) (end 60.33 65.33) (width 0.25) (layer "B.Cu") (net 24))
 (segment (start 60.33 65.33) (end 60.3 65.3) (width 0.25) (layer "B.Cu") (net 24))
 (segment (start 63.17 62.79) (end 60.31 62.79) (width 0.25) (layer "B.Cu") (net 25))
 (segment (start 60.31 62.79) (end 60.3 62.8) (width 0.25) (layer "B.Cu") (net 25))
 (segment (start 60.35 60.25) (end 60.3 60.3) (width 0.25) (layer "B.Cu") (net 26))
 (segment (start 63.17 60.25) (end 60.35 60.25) (width 0.25) (layer "B.Cu") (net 26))
 (segment (start 63.17 57.71) (end 60.31 57.71) (width 0.25) (layer "B.Cu") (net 27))
 (segment (start 60.31 57.71) (end 60.3 57.7) (width 0.25) (layer "B.Cu") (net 27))
 (segment (start 63.17 55.17) (end 60.33 55.17) (width 0.25) (layer "B.Cu") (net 28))
 (segment (start 60.33 55.17) (end 60.3 55.2) (width 0.25) (layer "B.Cu") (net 28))
 (segment (start 63.17 52.63) (end 60.33 52.63) (width 0.25) (layer "B.Cu") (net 29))
 (segment (start 60.33 52.63) (end 60.3 52.6) (width 0.25) (layer "B.Cu") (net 29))
 (segment (start 63.17 50.09) (end 60.31 50.09) (width 0.25) (layer "B.Cu") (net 30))
 (segment (start 60.31 50.09) (end 60.3 50.1) (width 0.25) (layer "B.Cu") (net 30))
 (segment (start 69.18 47.525) (end 71.98 47.525) (width 0.25) (layer "F.Cu") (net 13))
 (segment (start 71.98 47.525) (end 72.005 47.5) (width 0.25) (layer "F.Cu") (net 13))
 (segment (start 69.18 50.065) (end 71.982857 50.065) (width 0.25) (layer "F.Cu") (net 15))
 (segment (start 71.982857 50.065) (end 72.005 50.042857) (width 0.25) (layer "F.Cu") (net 15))
 (segment (start 69.18 52.605) (end 71.985714 52.605) (width 0.25) (layer "F.Cu") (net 3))
 (segment (start 71.985714 52.605) (end 72.005 52.585714) (width 0.25) (layer "F.Cu") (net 3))
 (segment (start 71.988571 55.145) (end 72.005 55.128571) (width 0.25) (layer "F.Cu") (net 31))
 (segment (start 69.18 55.145) (end 71.988571 55.145) (width 0.25) (layer "F.Cu") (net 31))
 (segment (start 69.18 57.685) (end 71.991428 57.685) (width 0.25) (layer "F.Cu") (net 11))
 (segment (start 71.991428 57.685) (end 72.005 57.671428) (width 0.25) (layer "F.Cu") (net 11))
 (segment (start 69.18 60.225) (end 71.994285 60.225) (width 0.25) (layer "F.Cu") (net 5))
 (segment (start 71.994285 60.225) (end 72.005 60.214285) (width 0.25) (layer "F.Cu") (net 5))
 (segment (start 69.18 62.765) (end 71.997142 62.765) (width 0.25) (layer "F.Cu") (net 20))
 (segment (start 71.997142 62.765) (end 72.005 62.757142) (width 0.25) (layer "F.Cu") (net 20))
 (segment (start 72 65.305) (end 72.005 65.3) (width 0.25) (layer "F.Cu") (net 9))
 (segment (start 69.18 65.305) (end 72 65.305) (width 0.25) (layer "F.Cu") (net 9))
 (segment (start 74.01 65.305) (end 76.8 65.305) (width 0.25) (layer "F.Cu") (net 10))
 (segment (start 74.005 65.3) (end 74.01 65.305) (width 0.25) (layer "F.Cu") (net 10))
 (segment (start 74.005 62.757142) (end 74.012858 62.765) (width 0.25) (layer "F.Cu") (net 21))
 (segment (start 74.012858 62.765) (end 76.8 62.765) (width 0.25) (layer "F.Cu") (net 21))
 (segment (start 74.005 60.214285) (end 74.015715 60.225) (width 0.25) (layer "F.Cu") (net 6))
 (segment (start 74.015715 60.225) (end 76.8 60.225) (width 0.25) (layer "F.Cu") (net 6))
 (segment (start 74.005 57.671428) (end 74.018572 57.685) (width 0.25) (layer "F.Cu") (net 12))
 (segment (start 74.018572 57.685) (end 76.8 57.685) (width 0.25) (layer "F.Cu") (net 12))
 (segment (start 74.021429 55.145) (end 76.8 55.145) (width 0.25) (layer "F.Cu") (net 32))
 (segment (start 74.005 55.128571) (end 74.021429 55.145) (width 0.25) (layer "F.Cu") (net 32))
 (segment (start 74.024286 52.605) (end 76.8 52.605) (width 0.25) (layer "F.Cu") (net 4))
 (segment (start 74.005 52.585714) (end 74.024286 52.605) (width 0.25) (layer "F.Cu") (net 4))
 (segment (start 74.005 50.042857) (end 74.027143 50.065) (width 0.25) (layer "F.Cu") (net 16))
 (segment (start 74.027143 50.065) (end 76.8 50.065) (width 0.25) (layer "F.Cu") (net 16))
 (segment (start 74.03 47.525) (end 76.8 47.525) (width 0.25) (layer "F.Cu") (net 14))
 (segment (start 74.005 47.5) (end 74.03 47.525) (width 0.25) (layer "F.Cu") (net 14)))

